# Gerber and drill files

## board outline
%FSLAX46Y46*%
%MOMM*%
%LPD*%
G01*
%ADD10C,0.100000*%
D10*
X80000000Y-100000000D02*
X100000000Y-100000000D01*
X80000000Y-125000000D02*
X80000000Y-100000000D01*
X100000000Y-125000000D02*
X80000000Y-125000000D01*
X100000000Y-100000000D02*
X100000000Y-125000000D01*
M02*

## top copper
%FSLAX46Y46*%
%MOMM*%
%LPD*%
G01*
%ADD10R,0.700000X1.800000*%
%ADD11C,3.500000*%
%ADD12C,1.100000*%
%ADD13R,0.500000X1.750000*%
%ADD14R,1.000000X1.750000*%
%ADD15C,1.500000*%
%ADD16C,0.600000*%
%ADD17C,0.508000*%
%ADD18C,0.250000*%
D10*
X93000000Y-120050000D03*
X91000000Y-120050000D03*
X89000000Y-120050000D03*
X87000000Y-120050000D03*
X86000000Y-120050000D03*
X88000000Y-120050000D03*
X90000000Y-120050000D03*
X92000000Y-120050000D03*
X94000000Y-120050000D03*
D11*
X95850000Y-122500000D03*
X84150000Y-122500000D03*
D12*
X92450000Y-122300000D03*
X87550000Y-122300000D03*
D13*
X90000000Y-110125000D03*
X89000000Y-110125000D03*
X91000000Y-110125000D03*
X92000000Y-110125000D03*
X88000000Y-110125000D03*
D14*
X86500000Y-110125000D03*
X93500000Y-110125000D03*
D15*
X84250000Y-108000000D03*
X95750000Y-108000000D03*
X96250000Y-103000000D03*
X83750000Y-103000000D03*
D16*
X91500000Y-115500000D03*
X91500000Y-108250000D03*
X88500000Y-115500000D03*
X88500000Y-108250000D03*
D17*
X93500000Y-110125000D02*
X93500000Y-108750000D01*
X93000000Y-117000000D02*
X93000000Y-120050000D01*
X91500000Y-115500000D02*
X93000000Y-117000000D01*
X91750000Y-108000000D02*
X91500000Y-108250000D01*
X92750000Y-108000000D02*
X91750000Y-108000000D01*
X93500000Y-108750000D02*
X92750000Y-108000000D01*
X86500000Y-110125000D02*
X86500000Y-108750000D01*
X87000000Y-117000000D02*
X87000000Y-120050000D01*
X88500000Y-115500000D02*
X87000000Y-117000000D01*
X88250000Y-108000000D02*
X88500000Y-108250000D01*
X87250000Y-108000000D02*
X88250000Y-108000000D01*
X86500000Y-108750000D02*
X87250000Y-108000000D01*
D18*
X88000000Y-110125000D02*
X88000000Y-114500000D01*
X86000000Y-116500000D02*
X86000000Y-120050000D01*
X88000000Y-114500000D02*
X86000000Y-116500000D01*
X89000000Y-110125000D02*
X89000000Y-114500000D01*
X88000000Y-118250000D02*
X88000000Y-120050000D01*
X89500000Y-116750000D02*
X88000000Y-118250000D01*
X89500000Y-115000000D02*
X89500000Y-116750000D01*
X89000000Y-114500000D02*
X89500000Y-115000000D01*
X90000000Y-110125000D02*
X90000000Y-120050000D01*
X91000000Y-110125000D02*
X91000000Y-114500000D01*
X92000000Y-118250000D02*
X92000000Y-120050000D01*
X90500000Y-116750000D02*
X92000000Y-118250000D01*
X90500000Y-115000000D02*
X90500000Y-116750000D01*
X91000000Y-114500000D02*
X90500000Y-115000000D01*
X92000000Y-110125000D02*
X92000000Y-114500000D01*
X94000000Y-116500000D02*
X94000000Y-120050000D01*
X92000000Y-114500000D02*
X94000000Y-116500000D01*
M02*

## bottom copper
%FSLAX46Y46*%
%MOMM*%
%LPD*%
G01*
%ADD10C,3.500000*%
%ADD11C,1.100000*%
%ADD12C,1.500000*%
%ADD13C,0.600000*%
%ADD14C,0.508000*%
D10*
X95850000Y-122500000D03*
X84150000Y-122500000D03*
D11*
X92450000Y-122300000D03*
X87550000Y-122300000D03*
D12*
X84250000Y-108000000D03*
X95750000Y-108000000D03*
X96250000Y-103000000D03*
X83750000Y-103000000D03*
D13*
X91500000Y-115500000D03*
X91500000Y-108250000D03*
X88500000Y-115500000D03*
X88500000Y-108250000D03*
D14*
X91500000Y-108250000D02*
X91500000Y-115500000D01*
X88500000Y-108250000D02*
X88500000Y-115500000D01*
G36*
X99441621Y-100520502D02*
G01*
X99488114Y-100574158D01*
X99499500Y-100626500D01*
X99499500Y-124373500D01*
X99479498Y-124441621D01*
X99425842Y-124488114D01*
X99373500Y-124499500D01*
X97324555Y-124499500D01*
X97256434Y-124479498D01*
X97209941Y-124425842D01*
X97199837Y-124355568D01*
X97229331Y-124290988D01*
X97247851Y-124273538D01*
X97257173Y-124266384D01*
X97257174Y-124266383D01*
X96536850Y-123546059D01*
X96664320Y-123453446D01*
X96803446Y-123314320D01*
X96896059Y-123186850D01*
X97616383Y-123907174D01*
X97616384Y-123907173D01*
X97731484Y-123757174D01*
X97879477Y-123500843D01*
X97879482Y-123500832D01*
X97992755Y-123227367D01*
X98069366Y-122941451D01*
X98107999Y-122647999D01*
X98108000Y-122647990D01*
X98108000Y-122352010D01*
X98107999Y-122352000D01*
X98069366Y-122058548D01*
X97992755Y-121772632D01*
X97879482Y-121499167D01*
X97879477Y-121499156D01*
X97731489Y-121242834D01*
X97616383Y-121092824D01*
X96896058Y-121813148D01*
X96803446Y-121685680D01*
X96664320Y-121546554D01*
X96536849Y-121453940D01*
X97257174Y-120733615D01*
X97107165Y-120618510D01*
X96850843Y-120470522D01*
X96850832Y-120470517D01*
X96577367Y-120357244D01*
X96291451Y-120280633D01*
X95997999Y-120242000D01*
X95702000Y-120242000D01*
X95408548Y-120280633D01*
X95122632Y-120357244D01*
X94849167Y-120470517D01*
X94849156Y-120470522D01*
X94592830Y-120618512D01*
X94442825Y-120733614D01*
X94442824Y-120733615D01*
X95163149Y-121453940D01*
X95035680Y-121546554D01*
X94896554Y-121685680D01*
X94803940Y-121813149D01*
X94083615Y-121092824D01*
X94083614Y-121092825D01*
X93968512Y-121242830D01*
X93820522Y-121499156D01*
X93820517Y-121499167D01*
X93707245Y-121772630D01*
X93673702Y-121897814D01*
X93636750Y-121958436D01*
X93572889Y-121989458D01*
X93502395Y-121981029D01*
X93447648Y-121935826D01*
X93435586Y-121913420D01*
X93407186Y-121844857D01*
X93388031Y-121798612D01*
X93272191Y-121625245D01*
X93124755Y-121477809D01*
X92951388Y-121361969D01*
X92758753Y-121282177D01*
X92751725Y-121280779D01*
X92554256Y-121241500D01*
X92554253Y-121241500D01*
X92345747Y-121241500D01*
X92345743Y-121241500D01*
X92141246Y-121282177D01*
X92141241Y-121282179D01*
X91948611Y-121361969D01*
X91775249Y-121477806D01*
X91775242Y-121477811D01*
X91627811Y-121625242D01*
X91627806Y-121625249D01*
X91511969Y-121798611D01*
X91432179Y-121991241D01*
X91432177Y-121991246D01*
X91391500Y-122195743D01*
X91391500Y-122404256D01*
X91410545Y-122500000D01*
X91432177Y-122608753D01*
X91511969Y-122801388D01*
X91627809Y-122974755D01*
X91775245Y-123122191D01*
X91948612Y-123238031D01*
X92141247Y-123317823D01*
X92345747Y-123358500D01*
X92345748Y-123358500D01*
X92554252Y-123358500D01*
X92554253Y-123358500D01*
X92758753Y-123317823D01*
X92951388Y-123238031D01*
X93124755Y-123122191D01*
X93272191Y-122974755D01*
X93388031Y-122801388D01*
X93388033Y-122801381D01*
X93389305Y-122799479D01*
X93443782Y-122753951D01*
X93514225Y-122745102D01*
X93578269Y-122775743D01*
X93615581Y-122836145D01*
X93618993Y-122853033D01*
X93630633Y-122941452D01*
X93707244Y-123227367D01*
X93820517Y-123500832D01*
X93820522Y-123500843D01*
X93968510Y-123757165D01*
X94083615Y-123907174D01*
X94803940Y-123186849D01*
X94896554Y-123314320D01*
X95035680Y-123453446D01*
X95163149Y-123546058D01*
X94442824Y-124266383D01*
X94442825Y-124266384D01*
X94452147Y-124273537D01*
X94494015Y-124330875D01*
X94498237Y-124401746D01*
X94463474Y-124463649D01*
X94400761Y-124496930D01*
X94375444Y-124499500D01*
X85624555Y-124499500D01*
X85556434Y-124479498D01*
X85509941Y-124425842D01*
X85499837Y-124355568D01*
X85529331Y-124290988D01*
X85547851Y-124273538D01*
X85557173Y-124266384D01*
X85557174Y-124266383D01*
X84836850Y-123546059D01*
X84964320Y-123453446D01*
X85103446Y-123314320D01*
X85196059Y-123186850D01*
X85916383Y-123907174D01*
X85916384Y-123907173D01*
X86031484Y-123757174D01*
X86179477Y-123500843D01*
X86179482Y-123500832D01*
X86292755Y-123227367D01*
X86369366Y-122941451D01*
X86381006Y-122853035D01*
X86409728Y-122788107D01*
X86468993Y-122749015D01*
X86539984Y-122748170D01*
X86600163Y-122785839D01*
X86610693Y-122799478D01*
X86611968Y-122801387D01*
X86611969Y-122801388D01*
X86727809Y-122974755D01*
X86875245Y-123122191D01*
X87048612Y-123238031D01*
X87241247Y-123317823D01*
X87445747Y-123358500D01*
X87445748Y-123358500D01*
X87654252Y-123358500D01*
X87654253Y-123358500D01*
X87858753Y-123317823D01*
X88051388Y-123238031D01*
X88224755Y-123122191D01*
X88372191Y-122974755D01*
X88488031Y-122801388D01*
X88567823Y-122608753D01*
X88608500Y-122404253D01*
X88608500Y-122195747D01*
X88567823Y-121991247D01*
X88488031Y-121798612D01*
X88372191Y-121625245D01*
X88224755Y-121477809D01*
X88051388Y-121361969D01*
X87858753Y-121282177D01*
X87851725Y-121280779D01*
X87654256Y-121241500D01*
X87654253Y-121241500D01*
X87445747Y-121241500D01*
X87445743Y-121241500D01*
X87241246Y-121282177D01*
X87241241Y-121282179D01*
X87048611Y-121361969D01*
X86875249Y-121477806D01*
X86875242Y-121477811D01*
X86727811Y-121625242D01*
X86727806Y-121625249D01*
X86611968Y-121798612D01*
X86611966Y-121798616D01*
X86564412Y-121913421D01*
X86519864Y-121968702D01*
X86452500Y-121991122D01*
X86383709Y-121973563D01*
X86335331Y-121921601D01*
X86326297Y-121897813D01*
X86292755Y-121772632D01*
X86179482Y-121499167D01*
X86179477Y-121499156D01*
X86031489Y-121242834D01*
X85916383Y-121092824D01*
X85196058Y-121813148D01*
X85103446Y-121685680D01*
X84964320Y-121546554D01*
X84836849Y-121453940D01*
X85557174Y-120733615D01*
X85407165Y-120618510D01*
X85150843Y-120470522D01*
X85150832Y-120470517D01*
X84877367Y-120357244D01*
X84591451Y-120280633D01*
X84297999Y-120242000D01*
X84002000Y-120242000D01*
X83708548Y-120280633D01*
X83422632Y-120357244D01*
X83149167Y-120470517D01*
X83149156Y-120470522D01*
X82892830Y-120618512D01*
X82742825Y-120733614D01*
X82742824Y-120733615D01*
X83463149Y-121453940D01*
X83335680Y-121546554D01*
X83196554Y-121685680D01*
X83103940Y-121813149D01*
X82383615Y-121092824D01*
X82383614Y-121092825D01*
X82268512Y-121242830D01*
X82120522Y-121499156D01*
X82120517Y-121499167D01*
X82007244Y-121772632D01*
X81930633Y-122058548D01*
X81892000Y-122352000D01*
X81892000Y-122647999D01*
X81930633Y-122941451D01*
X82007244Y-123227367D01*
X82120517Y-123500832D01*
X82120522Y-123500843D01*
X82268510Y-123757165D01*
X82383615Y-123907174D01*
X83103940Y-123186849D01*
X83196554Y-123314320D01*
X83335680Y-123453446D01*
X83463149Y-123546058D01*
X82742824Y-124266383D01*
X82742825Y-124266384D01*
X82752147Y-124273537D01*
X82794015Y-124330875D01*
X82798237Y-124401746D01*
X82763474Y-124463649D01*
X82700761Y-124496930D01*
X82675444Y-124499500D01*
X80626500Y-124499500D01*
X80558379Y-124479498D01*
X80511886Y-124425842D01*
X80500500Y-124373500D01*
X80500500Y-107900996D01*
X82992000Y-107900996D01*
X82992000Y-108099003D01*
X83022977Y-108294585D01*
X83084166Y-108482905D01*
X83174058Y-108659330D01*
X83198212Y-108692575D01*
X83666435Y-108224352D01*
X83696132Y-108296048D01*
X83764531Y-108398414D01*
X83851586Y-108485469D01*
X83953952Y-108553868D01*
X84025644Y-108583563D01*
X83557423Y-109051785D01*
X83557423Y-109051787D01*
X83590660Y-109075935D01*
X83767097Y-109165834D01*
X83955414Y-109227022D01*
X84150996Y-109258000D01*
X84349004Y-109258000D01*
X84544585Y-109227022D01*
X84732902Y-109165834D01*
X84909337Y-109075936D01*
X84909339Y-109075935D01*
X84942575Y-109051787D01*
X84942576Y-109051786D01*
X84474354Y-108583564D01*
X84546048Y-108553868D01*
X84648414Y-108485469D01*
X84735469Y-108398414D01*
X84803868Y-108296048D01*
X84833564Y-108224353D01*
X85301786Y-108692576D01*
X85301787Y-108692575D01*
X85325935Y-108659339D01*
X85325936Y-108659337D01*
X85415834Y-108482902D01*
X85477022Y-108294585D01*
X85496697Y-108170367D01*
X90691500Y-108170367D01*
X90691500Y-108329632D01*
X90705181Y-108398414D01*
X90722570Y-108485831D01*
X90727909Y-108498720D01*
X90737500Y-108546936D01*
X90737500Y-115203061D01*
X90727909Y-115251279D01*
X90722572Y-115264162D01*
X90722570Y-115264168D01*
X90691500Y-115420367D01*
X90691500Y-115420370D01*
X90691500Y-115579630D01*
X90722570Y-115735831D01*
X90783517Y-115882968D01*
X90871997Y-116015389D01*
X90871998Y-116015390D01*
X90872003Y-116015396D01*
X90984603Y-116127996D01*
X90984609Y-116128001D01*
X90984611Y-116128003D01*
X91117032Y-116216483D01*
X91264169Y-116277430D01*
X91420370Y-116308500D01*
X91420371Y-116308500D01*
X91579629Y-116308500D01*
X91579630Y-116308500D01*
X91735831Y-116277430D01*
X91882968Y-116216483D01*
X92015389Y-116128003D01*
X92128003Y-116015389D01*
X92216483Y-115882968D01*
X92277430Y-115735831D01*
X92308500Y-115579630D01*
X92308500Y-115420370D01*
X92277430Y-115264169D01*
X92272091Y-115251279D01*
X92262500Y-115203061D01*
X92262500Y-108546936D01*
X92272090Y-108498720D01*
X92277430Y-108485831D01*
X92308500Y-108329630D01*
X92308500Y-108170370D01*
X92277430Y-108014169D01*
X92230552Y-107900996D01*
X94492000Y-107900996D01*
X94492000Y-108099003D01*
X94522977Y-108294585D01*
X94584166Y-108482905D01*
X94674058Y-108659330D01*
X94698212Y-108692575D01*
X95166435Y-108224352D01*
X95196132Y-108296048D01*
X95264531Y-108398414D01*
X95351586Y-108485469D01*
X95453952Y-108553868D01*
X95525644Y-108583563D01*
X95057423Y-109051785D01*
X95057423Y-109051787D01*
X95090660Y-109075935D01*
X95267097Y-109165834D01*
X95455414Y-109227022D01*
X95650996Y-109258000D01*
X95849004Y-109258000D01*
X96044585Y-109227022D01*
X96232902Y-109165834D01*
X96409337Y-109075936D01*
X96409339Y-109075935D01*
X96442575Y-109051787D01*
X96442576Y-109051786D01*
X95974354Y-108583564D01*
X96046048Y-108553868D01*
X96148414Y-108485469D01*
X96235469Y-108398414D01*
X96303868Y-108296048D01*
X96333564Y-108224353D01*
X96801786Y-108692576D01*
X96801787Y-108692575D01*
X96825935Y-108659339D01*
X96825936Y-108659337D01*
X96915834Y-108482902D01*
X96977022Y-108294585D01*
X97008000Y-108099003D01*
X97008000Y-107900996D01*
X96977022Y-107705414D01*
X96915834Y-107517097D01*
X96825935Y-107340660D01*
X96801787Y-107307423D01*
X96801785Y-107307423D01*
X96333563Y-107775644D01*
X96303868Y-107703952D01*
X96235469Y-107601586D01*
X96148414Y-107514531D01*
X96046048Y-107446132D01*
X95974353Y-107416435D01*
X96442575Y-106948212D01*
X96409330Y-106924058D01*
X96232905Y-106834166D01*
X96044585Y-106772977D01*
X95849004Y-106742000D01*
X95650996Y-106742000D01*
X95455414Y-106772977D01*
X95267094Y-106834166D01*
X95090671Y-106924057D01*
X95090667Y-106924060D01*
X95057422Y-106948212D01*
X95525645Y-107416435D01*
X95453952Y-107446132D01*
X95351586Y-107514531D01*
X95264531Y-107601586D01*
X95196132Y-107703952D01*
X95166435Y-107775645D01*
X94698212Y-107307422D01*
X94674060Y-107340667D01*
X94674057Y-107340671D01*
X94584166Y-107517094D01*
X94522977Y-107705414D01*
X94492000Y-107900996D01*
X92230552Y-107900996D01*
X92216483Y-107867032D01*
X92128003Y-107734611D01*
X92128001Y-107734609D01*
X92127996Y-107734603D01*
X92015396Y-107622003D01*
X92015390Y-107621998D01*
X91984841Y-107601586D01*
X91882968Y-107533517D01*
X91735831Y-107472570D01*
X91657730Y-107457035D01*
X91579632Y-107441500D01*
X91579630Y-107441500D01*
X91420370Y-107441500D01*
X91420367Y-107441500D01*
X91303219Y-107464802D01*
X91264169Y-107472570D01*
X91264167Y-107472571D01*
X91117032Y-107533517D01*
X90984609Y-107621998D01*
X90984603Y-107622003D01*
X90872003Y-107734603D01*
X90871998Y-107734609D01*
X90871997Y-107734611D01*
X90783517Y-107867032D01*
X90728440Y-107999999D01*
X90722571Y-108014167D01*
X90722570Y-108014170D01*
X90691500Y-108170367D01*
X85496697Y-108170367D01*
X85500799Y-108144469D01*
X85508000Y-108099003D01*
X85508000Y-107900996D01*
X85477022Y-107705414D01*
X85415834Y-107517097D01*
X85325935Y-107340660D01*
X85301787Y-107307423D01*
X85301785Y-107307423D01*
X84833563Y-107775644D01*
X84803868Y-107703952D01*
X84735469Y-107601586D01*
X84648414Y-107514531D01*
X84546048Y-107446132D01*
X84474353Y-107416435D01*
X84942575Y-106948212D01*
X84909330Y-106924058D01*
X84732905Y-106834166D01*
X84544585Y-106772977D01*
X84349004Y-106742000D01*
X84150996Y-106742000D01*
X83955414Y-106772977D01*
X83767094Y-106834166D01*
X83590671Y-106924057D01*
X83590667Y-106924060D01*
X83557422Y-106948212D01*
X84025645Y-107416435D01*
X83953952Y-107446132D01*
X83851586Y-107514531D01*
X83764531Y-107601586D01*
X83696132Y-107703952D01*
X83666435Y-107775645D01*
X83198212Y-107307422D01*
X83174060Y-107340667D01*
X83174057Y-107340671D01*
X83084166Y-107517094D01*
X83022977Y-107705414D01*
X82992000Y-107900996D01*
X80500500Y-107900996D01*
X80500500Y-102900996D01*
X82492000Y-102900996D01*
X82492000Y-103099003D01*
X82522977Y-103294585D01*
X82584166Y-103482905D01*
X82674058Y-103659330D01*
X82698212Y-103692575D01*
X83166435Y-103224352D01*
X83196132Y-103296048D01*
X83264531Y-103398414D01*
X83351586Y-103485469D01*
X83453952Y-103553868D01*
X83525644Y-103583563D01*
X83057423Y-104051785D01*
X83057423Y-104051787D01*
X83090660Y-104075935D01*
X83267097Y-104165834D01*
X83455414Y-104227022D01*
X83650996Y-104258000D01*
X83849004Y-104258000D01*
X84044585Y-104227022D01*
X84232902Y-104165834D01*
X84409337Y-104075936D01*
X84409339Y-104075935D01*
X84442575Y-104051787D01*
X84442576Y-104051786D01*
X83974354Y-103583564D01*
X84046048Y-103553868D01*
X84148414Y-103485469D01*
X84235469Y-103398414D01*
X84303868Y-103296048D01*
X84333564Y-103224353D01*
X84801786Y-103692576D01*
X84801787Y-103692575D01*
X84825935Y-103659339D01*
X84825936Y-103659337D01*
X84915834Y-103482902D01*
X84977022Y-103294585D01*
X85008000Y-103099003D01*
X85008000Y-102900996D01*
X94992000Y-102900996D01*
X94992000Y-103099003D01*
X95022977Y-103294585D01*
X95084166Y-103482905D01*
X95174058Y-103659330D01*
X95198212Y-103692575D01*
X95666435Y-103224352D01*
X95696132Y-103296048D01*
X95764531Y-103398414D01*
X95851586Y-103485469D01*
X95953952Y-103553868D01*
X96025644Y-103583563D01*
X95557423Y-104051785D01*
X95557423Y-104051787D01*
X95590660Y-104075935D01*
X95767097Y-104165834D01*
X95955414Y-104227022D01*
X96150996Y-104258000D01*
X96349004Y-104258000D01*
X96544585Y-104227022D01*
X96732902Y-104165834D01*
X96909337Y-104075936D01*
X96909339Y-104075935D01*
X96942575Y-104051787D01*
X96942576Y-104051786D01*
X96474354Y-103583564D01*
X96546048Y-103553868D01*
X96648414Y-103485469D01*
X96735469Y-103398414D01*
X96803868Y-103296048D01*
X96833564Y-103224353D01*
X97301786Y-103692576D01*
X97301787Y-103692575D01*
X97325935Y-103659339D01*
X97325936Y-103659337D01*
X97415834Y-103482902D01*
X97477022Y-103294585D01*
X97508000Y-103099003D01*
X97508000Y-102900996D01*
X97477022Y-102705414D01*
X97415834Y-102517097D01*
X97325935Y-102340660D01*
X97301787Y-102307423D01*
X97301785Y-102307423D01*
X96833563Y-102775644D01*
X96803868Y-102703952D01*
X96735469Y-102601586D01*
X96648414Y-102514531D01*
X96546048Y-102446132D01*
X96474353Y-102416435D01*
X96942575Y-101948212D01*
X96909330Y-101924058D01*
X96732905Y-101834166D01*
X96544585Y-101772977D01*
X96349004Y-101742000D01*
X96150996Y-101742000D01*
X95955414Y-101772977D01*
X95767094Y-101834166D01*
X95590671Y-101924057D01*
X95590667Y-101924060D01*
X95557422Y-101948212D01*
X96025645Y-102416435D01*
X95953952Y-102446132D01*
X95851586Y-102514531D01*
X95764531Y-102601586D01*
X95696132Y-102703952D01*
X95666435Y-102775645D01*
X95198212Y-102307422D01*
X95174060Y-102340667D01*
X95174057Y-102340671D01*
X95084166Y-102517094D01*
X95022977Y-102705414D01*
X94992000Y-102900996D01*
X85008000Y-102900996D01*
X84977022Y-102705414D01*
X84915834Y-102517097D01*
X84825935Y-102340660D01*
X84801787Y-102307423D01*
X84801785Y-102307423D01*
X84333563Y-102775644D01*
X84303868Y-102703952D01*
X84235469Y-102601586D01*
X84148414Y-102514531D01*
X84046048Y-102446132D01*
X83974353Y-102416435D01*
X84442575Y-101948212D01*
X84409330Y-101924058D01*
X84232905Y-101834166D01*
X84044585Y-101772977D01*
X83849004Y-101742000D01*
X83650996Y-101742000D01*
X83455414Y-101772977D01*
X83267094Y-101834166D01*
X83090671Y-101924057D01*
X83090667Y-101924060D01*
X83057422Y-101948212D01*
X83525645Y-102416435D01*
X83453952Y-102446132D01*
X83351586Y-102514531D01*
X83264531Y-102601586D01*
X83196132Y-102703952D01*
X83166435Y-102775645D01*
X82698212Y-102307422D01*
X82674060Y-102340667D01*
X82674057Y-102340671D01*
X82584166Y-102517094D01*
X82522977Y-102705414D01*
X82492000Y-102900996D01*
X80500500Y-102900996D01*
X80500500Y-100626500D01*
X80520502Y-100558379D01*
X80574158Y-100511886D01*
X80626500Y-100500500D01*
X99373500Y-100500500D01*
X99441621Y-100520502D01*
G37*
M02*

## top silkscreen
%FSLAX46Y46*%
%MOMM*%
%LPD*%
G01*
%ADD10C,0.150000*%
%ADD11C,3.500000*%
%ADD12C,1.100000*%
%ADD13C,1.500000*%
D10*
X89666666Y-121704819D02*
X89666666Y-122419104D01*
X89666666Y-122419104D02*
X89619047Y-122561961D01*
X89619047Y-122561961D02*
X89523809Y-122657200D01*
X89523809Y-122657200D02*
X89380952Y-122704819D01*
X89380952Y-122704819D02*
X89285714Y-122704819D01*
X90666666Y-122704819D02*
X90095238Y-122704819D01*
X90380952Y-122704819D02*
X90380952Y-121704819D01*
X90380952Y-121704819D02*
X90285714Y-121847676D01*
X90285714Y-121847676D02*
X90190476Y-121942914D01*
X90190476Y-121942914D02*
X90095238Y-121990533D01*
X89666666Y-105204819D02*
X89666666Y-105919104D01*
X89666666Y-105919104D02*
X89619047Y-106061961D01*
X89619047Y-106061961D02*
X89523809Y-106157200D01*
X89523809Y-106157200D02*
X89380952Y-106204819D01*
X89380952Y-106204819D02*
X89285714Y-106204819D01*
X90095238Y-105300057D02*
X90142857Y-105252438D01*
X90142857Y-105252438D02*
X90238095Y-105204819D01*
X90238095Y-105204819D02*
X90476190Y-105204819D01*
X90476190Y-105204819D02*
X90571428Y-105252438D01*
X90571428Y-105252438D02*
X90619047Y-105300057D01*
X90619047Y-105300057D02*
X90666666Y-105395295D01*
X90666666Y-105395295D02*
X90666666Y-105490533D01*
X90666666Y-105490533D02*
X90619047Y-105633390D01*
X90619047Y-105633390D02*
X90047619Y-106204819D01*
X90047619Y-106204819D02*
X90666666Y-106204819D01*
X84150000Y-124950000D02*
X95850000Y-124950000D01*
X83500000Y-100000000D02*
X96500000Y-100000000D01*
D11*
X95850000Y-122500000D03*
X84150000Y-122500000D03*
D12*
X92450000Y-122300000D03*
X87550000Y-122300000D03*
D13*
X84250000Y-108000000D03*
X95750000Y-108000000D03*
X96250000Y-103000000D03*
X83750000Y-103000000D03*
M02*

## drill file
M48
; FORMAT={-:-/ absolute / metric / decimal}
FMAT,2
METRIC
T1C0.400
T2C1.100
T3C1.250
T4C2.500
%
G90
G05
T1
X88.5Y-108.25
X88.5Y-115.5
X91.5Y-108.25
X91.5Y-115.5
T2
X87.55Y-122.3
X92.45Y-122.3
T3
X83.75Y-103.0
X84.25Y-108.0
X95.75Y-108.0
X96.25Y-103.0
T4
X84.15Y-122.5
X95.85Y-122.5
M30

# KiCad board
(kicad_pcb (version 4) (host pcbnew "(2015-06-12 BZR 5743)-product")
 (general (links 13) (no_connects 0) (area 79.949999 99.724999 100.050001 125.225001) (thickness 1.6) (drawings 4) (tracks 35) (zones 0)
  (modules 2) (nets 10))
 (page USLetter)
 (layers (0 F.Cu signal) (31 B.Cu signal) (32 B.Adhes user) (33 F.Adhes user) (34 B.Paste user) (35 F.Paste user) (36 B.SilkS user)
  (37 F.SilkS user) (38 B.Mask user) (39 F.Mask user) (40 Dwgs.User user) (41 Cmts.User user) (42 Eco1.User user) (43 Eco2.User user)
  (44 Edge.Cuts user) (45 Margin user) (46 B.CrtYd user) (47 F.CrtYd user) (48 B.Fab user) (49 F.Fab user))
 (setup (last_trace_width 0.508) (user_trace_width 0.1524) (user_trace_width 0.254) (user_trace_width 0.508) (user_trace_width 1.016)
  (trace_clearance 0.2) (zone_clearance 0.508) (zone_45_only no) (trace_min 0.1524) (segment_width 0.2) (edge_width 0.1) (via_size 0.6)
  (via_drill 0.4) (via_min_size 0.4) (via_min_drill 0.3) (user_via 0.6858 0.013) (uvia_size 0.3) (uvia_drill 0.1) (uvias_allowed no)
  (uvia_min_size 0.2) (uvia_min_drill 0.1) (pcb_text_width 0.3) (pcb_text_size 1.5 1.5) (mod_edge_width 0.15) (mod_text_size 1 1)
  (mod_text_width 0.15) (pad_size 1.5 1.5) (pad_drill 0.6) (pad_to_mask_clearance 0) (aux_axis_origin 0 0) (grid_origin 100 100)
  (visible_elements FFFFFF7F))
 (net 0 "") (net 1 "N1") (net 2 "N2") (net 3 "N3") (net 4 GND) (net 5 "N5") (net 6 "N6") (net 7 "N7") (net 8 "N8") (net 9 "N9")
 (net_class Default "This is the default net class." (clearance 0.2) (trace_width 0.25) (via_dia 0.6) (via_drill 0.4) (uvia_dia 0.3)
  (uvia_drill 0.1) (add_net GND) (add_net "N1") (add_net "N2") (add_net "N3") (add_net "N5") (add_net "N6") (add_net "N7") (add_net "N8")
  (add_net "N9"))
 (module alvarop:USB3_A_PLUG (layer F.Cu) (at 90 122.3)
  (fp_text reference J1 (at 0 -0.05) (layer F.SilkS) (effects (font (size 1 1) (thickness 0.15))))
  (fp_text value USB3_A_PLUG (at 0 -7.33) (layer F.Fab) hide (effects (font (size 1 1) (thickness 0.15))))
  (fp_line (start -5.85 2.65) (end 5.85 2.65) (layer F.SilkS) (width 0.15))
  (pad 1 smd rect (at 3 -2.25) (size 0.7 1.8) (layers F.Cu F.Paste F.Mask) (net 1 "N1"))
  (pad 2 smd rect (at 1 -2.25) (size 0.7 1.8) (layers F.Cu F.Paste F.Mask) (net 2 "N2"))
  (pad 3 smd rect (at -1 -2.25) (size 0.7 1.8) (layers F.Cu F.Paste F.Mask) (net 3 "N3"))
  (pad 4 smd rect (at -3 -2.25) (size 0.7 1.8) (layers F.Cu F.Paste F.Mask) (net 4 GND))
  (pad 5 smd rect (at -4 -2.25) (size 0.7 1.8) (layers F.Cu F.Paste F.Mask) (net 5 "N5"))
  (pad 6 smd rect (at -2 -2.25) (size 0.7 1.8) (layers F.Cu F.Paste F.Mask) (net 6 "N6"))
  (pad 7 smd rect (at 0 -2.25) (size 0.7 1.8) (layers F.Cu F.Paste F.Mask) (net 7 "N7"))
  (pad 8 smd rect (at 2 -2.25) (size 0.7 1.8) (layers F.Cu F.Paste F.Mask) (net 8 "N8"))
  (pad 9 smd rect (at 4 -2.25) (size 0.7 1.8) (layers F.Cu F.Paste F.Mask) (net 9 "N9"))
  (pad 10 thru_hole circle (at 5.85 0.2) (size 3.5 3.5) (drill 2.5) (layers *.Cu *.Mask F.SilkS) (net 4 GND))
  (pad 10 thru_hole circle (at -5.85 0.2) (size 3.5 3.5) (drill 2.5) (layers *.Cu *.Mask F.SilkS) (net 4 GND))
  (pad "" thru_hole circle (at 2.45 0) (size 1.1 1.1) (drill 1.1) (layers *.Cu *.Mask F.SilkS))
  (pad "" thru_hole circle (at -2.45 0) (size 1.1 1.1) (drill 1.1) (layers *.Cu *.Mask F.SilkS)))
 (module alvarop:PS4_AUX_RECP (layer F.Cu) (at 90 110 180)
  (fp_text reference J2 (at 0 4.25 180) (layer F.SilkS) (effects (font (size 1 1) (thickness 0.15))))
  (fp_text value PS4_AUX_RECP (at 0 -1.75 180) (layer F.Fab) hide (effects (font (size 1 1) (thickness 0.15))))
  (fp_line (start 6.5 10) (end -6.5 10) (layer F.SilkS) (width 0.15))
  (pad 4 smd rect (at 0 -0.125 180) (size 0.5 1.75) (layers F.Cu F.Paste F.Mask) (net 7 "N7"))
  (pad 3 smd rect (at 1 -0.125 180) (size 0.5 1.75) (layers F.Cu F.Paste F.Mask) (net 6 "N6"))
  (pad 5 smd rect (at -1 -0.125 180) (size 0.5 1.75) (layers F.Cu F.Paste F.Mask) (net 8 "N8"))
  (pad 6 smd rect (at -2 -0.125 180) (size 0.5 1.75) (layers F.Cu F.Paste F.Mask) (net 9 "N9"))
  (pad 2 smd rect (at 2 -0.125 180) (size 0.5 1.75) (layers F.Cu F.Paste F.Mask) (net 5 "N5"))
  (pad 1 smd rect (at 3.5 -0.125 180) (size 1 1.75) (layers F.Cu F.Paste F.Mask) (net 4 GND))
  (pad 7 smd rect (at -3.5 -0.125 180) (size 1 1.75) (layers F.Cu F.Paste F.Mask) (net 1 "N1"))
  (pad 8 thru_hole circle (at 5.75 2 180) (size 1.5 1.5) (drill 1.25) (layers *.Cu *.Mask F.SilkS) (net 4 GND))
  (pad 8 thru_hole circle (at -5.75 2 180) (size 1.5 1.5) (drill 1.25) (layers *.Cu *.Mask F.SilkS) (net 4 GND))
  (pad 8 thru_hole circle (at -6.25 7 180) (size 1.5 1.5) (drill 1.25) (layers *.Cu *.Mask F.SilkS) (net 4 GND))
  (pad 8 thru_hole circle (at 6.25 7 180) (size 1.5 1.5) (drill 1.25) (layers *.Cu *.Mask F.SilkS) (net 4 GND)))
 (gr_line (start 80 100) (end 100 100) (angle 90) (layer Edge.Cuts) (width 0.1))
 (gr_line (start 80 125) (end 80 100) (angle 90) (layer Edge.Cuts) (width 0.1))
 (gr_line (start 100 125) (end 80 125) (angle 90) (layer Edge.Cuts) (width 0.1))
 (gr_line (start 100 100) (end 100 125) (angle 90) (layer Edge.Cuts) (width 0.1))
 (segment (start 93.5 110.125) (end 93.5 108.75) (width 0.508) (layer F.Cu) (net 1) (status 400000))
 (segment (start 93 117) (end 93 120.05) (width 0.508) (layer F.Cu) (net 1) (status 800000))
 (segment (start 91.5 115.5) (end 93 117) (width 0.508) (layer F.Cu) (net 1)) (via (at 91.5 115.5) (size 0.6) (layers F.Cu B.Cu) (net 1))
 (segment (start 91.5 108.25) (end 91.5 115.5) (width 0.508) (layer B.Cu) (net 1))
 (via (at 91.5 108.25) (size 0.6) (layers F.Cu B.Cu) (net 1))
 (segment (start 91.75 108) (end 91.5 108.25) (width 0.508) (layer F.Cu) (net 1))
 (segment (start 92.75 108) (end 91.75 108) (width 0.508) (layer F.Cu) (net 1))
 (segment (start 93.5 108.75) (end 92.75 108) (width 0.508) (layer F.Cu) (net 1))
 (segment (start 86.5 110.125) (end 86.5 108.75) (width 0.508) (layer F.Cu) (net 4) (status 400000))
 (segment (start 87 117) (end 87 120.05) (width 0.508) (layer F.Cu) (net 4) (status 800000))
 (segment (start 88.5 115.5) (end 87 117) (width 0.508) (layer F.Cu) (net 4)) (via (at 88.5 115.5) (size 0.6) (layers F.Cu B.Cu) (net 4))
 (segment (start 88.5 108.25) (end 88.5 115.5) (width 0.508) (layer B.Cu) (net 4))
 (via (at 88.5 108.25) (size 0.6) (layers F.Cu B.Cu) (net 4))
 (segment (start 88.25 108) (end 88.5 108.25) (width 0.508) (layer F.Cu) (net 4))
 (segment (start 87.25 108) (end 88.25 108) (width 0.508) (layer F.Cu) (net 4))
 (segment (start 86.5 108.75) (end 87.25 108) (width 0.508) (layer F.Cu) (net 4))
 (segment (start 88 110.125) (end 88 114.5) (width 0.25) (layer F.Cu) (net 5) (status 400000))
 (segment (start 86 116.5) (end 86 120.05) (width 0.25) (layer F.Cu) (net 5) (status 800000))
 (segment (start 88 114.5) (end 86 116.5) (width 0.25) (layer F.Cu) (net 5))
 (segment (start 89 110.125) (end 89 114.5) (width 0.25) (layer F.Cu) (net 6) (status 400000))
 (segment (start 88 118.25) (end 88 120.05) (width 0.25) (layer F.Cu) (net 6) (status 800000))
 (segment (start 89.5 116.75) (end 88 118.25) (width 0.25) (layer F.Cu) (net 6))
 (segment (start 89.5 115) (end 89.5 116.75) (width 0.25) (layer F.Cu) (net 6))
 (segment (start 89 114.5) (end 89.5 115) (width 0.25) (layer F.Cu) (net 6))
 (segment (start 90 110.125) (end 90 120.05) (width 0.25) (layer F.Cu) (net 7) (status C00000))
 (segment (start 91 110.125) (end 91 114.5) (width 0.25) (layer F.Cu) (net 8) (status 400000))
 (segment (start 92 118.25) (end 92 120.05) (width 0.25) (layer F.Cu) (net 8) (status 800000))
 (segment (start 90.5 116.75) (end 92 118.25) (width 0.25) (layer F.Cu) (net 8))
 (segment (start 90.5 115) (end 90.5 116.75) (width 0.25) (layer F.Cu) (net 8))
 (segment (start 91 114.5) (end 90.5 115) (width 0.25) (layer F.Cu) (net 8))
 (segment (start 92 110.125) (end 92 114.5) (width 0.25) (layer F.Cu) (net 9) (status 400000))
 (segment (start 94 116.5) (end 94 120.05) (width 0.25) (layer F.Cu) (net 9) (status 800000))
 (segment (start 92 114.5) (end 94 116.5) (width 0.25) (layer F.Cu) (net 9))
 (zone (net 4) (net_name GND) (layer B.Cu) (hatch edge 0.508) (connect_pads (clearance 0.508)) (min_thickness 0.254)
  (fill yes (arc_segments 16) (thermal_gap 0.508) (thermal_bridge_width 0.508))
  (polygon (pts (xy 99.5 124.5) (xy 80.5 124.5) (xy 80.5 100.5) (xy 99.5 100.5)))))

